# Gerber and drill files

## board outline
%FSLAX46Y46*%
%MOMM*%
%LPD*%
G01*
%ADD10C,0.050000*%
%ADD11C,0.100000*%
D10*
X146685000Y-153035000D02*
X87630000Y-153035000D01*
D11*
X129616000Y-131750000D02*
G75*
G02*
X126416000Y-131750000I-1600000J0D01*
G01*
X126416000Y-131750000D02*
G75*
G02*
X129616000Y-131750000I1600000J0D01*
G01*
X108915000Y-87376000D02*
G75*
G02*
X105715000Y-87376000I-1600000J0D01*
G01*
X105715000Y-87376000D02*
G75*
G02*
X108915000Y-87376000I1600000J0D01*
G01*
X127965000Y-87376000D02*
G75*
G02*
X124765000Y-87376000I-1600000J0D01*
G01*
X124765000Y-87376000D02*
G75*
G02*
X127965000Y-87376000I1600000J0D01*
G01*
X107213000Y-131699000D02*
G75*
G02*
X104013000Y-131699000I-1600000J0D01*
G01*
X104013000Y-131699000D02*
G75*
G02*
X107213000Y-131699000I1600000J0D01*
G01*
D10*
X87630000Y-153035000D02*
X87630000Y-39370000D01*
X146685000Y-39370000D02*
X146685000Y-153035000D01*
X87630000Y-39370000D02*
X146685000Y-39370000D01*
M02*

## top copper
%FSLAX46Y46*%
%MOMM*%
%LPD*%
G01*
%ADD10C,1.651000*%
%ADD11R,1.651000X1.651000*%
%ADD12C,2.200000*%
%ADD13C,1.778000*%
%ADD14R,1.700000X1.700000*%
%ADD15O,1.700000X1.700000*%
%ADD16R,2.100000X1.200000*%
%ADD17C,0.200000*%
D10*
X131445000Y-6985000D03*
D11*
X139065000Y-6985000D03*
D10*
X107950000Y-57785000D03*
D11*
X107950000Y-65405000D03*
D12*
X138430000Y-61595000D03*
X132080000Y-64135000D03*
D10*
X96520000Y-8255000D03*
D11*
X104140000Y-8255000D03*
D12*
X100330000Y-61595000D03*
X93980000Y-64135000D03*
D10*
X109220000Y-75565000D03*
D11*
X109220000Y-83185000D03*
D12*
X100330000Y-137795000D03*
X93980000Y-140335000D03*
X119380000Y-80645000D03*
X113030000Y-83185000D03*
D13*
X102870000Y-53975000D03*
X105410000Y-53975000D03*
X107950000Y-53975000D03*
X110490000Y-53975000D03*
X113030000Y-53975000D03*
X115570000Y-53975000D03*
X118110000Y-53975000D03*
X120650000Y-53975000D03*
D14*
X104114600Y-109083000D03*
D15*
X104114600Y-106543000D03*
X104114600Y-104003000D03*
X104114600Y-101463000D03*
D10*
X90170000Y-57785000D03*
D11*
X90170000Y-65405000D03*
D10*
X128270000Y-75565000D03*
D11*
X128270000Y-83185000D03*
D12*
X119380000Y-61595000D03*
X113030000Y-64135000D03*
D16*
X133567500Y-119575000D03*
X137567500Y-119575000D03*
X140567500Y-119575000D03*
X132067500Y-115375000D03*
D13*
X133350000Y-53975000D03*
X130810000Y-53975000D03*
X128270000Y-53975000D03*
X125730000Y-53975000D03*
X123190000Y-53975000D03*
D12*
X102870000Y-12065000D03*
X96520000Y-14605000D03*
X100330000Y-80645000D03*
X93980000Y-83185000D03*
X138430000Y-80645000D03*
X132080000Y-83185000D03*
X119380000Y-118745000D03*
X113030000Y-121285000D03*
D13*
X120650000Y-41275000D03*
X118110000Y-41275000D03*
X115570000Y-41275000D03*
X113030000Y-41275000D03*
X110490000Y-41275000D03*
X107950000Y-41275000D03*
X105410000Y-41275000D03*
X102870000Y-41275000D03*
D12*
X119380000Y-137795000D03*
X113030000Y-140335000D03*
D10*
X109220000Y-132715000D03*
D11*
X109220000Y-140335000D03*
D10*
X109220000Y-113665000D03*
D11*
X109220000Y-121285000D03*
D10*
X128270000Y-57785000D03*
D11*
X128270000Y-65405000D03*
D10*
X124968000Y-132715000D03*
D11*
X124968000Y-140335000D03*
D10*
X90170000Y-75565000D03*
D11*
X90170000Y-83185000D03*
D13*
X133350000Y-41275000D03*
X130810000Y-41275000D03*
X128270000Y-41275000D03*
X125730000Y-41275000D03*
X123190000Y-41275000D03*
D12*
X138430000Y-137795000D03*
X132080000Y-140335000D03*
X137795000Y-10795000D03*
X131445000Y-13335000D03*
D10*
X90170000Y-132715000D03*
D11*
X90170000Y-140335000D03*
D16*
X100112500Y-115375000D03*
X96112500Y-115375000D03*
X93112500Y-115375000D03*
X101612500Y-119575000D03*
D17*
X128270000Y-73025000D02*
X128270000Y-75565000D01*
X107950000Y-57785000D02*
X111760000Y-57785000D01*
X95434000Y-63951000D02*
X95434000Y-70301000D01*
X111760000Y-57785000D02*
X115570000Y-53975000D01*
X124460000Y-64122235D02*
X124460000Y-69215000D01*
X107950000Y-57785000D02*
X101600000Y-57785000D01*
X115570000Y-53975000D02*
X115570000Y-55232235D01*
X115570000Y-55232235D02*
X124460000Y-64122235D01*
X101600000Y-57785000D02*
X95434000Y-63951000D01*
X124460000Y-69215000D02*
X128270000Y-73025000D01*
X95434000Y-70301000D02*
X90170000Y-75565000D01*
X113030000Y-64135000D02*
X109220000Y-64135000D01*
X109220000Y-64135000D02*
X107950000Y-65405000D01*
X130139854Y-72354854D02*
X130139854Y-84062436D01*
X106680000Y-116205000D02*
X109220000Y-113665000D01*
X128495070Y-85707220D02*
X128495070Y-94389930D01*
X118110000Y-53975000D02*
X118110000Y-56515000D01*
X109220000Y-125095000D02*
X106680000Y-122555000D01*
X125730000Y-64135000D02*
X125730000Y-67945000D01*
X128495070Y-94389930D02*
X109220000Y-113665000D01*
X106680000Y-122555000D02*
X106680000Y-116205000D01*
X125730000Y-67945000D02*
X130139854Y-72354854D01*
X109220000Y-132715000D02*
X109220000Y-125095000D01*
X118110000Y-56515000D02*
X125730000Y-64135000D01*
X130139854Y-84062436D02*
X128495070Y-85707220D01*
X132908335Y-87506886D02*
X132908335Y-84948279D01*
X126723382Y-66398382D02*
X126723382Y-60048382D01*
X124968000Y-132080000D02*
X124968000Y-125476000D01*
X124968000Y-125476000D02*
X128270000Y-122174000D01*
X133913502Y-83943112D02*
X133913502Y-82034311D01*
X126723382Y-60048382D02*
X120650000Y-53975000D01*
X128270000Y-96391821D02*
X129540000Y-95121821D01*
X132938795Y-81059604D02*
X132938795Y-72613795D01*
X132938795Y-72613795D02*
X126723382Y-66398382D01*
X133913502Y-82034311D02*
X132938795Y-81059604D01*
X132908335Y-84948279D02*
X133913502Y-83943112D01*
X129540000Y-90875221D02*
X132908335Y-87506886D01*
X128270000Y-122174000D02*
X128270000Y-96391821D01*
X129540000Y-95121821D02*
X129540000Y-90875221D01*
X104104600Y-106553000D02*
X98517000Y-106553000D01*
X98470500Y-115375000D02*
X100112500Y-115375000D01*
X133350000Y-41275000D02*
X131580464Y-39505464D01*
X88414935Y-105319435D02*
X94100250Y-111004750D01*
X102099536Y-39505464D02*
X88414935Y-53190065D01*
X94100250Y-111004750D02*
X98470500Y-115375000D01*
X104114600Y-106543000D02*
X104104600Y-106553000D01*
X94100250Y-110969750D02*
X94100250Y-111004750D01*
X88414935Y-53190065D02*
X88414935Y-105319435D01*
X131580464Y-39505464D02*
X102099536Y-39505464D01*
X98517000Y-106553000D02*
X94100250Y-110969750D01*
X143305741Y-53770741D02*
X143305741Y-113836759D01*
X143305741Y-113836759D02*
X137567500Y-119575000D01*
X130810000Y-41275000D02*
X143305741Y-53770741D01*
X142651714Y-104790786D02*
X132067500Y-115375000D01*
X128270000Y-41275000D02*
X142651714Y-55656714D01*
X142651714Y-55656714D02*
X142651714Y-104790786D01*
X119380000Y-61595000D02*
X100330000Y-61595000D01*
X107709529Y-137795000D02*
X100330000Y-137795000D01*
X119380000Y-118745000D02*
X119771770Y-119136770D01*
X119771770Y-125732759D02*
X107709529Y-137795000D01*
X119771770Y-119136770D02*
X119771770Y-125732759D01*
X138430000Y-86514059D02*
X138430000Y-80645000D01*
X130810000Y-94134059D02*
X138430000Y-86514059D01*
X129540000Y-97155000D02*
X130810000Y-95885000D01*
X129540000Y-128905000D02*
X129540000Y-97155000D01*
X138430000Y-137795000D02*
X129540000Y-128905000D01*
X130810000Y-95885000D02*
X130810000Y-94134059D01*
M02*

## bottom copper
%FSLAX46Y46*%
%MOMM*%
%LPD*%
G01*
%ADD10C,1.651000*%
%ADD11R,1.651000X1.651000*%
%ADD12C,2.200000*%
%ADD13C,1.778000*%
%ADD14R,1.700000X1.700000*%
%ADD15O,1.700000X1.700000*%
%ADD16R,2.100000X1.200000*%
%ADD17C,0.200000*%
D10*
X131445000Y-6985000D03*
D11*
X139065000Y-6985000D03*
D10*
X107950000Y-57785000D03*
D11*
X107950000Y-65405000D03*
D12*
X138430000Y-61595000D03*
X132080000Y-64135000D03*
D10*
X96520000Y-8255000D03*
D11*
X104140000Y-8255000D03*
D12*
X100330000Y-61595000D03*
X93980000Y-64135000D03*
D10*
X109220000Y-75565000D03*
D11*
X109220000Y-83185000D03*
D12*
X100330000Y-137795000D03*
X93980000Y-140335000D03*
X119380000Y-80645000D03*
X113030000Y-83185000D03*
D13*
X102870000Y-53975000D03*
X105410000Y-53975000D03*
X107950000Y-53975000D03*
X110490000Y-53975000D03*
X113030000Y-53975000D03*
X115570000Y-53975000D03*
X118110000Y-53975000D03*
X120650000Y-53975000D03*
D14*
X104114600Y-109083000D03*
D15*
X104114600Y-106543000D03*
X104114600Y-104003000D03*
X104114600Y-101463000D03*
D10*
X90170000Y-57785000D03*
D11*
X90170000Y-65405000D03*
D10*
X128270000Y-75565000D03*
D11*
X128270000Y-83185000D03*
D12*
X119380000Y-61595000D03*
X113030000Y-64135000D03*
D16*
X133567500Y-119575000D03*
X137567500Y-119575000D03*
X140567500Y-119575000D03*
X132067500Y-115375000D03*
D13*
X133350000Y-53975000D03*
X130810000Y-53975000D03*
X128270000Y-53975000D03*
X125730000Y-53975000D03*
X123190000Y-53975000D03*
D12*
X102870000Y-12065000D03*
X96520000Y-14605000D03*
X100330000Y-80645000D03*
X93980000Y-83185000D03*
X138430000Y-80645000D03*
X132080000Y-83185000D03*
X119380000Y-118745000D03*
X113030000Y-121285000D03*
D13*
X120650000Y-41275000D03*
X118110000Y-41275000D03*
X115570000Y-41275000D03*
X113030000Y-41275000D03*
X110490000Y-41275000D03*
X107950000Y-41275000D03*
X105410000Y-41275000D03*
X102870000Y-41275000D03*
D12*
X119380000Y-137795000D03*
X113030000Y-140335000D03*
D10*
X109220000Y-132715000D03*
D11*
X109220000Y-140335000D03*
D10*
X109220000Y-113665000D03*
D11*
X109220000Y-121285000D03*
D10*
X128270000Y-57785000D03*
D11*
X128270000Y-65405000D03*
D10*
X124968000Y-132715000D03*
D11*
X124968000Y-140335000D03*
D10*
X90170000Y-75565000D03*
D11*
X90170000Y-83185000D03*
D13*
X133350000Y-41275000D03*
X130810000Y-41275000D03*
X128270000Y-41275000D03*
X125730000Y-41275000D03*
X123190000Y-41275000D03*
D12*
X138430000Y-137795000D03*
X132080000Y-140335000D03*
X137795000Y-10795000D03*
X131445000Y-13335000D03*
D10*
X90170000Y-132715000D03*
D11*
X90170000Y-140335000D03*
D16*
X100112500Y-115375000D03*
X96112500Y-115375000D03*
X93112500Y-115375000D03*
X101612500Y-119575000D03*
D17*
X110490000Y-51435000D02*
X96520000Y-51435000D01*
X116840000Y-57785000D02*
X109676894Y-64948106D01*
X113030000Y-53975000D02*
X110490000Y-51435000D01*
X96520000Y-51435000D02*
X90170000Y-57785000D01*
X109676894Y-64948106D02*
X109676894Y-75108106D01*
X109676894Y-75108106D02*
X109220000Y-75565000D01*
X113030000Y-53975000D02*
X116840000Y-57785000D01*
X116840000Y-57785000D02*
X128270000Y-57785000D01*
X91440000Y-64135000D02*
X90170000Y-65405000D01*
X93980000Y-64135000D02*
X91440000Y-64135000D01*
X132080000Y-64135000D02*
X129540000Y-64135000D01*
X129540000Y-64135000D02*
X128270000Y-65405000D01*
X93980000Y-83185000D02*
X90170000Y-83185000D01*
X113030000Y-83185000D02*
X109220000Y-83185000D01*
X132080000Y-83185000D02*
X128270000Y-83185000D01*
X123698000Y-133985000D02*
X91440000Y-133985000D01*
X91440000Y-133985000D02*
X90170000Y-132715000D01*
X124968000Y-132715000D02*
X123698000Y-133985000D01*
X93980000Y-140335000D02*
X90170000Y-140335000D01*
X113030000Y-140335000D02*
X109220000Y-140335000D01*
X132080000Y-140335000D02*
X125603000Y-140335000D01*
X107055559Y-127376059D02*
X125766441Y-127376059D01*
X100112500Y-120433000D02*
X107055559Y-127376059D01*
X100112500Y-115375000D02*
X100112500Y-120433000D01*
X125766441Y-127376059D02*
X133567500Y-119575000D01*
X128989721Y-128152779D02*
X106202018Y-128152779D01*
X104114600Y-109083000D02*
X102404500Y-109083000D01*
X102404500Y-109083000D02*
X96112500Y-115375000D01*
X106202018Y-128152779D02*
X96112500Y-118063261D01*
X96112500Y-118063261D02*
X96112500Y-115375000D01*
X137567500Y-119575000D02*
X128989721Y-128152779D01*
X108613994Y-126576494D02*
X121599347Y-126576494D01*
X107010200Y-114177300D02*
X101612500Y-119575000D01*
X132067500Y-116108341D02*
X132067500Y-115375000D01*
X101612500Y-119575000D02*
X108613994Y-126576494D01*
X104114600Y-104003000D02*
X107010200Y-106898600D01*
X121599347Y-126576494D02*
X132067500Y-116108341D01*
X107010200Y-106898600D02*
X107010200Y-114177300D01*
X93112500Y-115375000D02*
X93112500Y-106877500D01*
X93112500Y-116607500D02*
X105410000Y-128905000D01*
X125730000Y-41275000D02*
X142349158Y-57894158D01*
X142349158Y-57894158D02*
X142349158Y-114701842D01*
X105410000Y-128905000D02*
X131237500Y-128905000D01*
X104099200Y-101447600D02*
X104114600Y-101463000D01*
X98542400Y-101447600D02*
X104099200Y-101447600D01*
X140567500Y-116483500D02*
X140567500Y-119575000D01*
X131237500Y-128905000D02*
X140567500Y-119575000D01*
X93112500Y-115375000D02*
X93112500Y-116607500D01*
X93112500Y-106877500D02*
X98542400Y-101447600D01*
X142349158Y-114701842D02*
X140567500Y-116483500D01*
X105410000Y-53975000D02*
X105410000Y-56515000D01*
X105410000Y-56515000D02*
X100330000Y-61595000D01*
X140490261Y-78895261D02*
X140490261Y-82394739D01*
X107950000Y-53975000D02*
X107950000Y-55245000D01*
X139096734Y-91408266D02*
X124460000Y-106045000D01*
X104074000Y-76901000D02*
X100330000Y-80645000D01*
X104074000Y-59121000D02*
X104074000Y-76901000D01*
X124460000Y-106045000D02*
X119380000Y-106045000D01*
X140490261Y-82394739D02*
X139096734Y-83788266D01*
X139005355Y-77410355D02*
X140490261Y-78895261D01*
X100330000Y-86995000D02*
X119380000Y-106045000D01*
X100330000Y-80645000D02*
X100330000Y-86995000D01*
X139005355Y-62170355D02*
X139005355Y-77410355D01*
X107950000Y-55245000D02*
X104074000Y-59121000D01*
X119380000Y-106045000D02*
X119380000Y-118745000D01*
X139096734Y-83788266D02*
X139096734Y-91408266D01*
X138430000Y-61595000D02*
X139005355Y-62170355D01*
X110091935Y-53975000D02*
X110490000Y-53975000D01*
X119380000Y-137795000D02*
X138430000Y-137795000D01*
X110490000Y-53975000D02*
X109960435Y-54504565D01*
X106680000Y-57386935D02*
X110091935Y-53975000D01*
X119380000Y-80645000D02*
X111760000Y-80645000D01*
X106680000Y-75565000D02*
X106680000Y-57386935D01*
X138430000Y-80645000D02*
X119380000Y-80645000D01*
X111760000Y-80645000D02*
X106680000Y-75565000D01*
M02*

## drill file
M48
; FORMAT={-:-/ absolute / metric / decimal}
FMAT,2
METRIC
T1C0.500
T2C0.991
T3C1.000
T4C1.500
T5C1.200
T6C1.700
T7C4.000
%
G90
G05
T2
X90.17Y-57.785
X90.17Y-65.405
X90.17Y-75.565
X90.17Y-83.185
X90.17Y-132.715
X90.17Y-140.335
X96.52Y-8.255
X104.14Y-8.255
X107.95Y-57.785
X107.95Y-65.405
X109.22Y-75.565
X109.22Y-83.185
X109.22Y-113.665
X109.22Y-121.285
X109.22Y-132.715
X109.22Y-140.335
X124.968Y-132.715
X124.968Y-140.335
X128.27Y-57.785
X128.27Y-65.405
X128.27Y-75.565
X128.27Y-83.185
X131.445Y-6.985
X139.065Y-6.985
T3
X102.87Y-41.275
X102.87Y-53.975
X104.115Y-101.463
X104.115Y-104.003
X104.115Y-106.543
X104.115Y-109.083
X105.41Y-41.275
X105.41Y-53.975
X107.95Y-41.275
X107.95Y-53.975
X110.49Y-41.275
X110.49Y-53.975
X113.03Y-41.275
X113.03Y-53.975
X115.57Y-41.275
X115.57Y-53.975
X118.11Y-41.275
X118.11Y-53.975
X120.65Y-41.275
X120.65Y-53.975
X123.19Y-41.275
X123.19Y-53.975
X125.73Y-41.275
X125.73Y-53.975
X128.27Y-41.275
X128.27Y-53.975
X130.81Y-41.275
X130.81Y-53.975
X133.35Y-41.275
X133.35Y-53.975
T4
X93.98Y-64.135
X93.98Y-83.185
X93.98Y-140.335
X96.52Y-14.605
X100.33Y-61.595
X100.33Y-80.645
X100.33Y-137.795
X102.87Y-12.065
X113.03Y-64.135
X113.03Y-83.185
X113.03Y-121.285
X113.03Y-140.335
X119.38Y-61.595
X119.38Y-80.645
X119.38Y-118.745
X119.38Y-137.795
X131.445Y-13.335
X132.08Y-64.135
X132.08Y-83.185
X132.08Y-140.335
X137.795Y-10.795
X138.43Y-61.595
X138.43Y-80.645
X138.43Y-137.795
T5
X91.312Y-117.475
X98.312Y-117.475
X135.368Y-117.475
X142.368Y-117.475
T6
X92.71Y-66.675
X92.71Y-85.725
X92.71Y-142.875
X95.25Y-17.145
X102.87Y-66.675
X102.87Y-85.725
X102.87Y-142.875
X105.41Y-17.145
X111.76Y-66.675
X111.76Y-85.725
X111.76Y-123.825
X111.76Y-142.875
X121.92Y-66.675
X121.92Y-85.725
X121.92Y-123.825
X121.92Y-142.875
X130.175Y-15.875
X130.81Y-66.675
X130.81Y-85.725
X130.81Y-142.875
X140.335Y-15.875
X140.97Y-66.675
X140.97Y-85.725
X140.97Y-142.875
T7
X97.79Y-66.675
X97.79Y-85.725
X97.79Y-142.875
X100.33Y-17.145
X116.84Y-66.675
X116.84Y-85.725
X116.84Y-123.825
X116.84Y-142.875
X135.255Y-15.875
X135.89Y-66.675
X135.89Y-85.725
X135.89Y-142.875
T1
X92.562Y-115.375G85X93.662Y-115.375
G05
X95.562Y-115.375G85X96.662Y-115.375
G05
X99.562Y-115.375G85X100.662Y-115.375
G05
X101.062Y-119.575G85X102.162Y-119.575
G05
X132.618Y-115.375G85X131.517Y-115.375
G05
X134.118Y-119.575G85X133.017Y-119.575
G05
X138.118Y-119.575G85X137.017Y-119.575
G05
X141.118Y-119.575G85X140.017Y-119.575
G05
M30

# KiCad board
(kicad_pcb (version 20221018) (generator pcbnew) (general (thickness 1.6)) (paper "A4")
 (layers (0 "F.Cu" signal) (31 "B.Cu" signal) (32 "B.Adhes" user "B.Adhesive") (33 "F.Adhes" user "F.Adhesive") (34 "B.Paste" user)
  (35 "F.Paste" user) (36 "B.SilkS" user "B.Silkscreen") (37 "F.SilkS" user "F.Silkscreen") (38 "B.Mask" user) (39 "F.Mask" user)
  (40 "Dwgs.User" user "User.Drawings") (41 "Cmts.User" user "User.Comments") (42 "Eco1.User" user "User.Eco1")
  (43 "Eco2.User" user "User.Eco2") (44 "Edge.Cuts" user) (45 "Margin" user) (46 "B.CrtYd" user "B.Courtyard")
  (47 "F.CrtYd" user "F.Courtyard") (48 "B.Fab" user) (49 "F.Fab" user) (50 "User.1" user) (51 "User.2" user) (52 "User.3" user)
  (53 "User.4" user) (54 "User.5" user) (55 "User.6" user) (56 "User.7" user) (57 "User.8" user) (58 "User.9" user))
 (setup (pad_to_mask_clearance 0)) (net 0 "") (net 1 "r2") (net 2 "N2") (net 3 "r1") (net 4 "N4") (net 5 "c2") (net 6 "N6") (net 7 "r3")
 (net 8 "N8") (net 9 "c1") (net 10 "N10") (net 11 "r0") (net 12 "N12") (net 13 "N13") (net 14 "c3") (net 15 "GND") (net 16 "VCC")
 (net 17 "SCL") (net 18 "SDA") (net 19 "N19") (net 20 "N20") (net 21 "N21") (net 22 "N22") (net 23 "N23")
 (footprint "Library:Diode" (layer "F.Cu") (at 135.255 6.985)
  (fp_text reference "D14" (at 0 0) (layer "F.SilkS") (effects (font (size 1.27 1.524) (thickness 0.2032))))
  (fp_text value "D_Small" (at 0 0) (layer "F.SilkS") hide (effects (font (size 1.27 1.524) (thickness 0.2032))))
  (pad "1" thru_hole circle (at -3.81 0) (size 1.651 1.651) (drill 0.9906) (layers "*.Cu" "*.SilkS" "*.Mask") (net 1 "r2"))
  (pad "2" thru_hole rect (at 3.81 0) (size 1.651 1.651) (drill 0.9906) (layers "*.Cu" "*.SilkS" "*.Mask") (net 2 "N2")))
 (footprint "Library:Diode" (layer "F.Cu") (at 107.95 61.595 -90)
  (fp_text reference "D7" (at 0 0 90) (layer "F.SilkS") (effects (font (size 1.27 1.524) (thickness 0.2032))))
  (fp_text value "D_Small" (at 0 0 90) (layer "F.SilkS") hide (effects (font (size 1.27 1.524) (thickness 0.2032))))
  (pad "1" thru_hole circle (at -3.81 0 270) (size 1.651 1.651) (drill 0.9906) (layers "*.Cu" "*.SilkS" "*.Mask") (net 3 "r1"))
  (pad "2" thru_hole rect (at 3.81 0 270) (size 1.651 1.651) (drill 0.9906) (layers "*.Cu" "*.SilkS" "*.Mask") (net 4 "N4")))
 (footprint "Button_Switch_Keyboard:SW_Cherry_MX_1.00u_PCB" (layer "F.Cu") (at 138.43 61.595)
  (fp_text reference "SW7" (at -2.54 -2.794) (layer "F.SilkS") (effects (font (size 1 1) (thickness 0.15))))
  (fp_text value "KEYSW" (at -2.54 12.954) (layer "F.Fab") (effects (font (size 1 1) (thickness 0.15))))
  (pad "" np_thru_hole circle (at -7.62 5.08) (size 1.7 1.7) (drill 1.7) (layers "*.Cu" "*.Mask"))
  (pad "" np_thru_hole circle (at -2.54 5.08) (size 4 4) (drill 4) (layers "*.Cu" "*.Mask"))
  (pad "" np_thru_hole circle (at 2.54 5.08) (size 1.7 1.7) (drill 1.7) (layers "*.Cu" "*.Mask"))
  (pad "1" thru_hole circle (at 0 0) (size 2.2 2.2) (drill 1.5) (layers "*.Cu" "*.Mask") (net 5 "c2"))
  (pad "2" thru_hole circle (at -6.35 2.54) (size 2.2 2.2) (drill 1.5) (layers "*.Cu" "*.Mask") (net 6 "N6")))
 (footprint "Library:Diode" (layer "F.Cu") (at 100.33 8.255)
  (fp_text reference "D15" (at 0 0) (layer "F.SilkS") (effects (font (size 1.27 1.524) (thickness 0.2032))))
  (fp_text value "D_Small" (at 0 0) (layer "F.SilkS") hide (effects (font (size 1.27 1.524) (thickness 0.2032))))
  (pad "1" thru_hole circle (at -3.81 0) (size 1.651 1.651) (drill 0.9906) (layers "*.Cu" "*.SilkS" "*.Mask") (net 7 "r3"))
  (pad "2" thru_hole rect (at 3.81 0) (size 1.651 1.651) (drill 0.9906) (layers "*.Cu" "*.SilkS" "*.Mask") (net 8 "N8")))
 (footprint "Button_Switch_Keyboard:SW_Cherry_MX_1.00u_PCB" (layer "F.Cu") (at 100.33 61.595)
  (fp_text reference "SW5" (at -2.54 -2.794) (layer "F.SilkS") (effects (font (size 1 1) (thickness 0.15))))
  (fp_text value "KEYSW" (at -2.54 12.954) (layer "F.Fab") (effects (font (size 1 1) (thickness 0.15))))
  (pad "" np_thru_hole circle (at -7.62 5.08) (size 1.7 1.7) (drill 1.7) (layers "*.Cu" "*.Mask"))
  (pad "" np_thru_hole circle (at -2.54 5.08) (size 4 4) (drill 4) (layers "*.Cu" "*.Mask"))
  (pad "" np_thru_hole circle (at 2.54 5.08) (size 1.7 1.7) (drill 1.7) (layers "*.Cu" "*.Mask"))
  (pad "1" thru_hole circle (at 0 0) (size 2.2 2.2) (drill 1.5) (layers "*.Cu" "*.Mask") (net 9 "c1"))
  (pad "2" thru_hole circle (at -6.35 2.54) (size 2.2 2.2) (drill 1.5) (layers "*.Cu" "*.Mask") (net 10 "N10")))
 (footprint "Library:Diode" (layer "F.Cu") (at 109.22 79.375 -90)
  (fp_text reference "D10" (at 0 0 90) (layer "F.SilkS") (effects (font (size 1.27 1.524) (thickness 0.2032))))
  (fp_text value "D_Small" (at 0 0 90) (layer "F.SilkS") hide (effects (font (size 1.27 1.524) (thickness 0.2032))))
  (pad "1" thru_hole circle (at -3.81 0 270) (size 1.651 1.651) (drill 0.9906) (layers "*.Cu" "*.SilkS" "*.Mask") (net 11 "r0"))
  (pad "2" thru_hole rect (at 3.81 0 270) (size 1.651 1.651) (drill 0.9906) (layers "*.Cu" "*.SilkS" "*.Mask") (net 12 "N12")))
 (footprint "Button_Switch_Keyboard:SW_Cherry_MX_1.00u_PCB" (layer "F.Cu") (at 100.33 137.795)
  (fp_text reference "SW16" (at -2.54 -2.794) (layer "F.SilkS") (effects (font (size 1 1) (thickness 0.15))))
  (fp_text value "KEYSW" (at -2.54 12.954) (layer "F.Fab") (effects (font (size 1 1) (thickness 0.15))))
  (pad "" np_thru_hole circle (at -7.62 5.08) (size 1.7 1.7) (drill 1.7) (layers "*.Cu" "*.Mask"))
  (pad "" np_thru_hole circle (at -2.54 5.08) (size 4 4) (drill 4) (layers "*.Cu" "*.Mask"))
  (pad "" np_thru_hole circle (at 2.54 5.08) (size 1.7 1.7) (drill 1.7) (layers "*.Cu" "*.Mask"))
  (pad "1" thru_hole circle (at 0 0) (size 2.2 2.2) (drill 1.5) (layers "*.Cu" "*.Mask") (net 5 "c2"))
  (pad "2" thru_hole circle (at -6.35 2.54) (size 2.2 2.2) (drill 1.5) (layers "*.Cu" "*.Mask") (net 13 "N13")))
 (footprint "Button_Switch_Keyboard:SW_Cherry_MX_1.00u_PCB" (layer "F.Cu") (at 119.38 80.645)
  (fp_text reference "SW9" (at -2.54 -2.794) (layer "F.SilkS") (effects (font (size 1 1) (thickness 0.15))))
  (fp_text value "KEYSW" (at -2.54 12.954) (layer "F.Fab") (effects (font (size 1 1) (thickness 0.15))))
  (pad "" np_thru_hole circle (at -7.62 5.08) (size 1.7 1.7) (drill 1.7) (layers "*.Cu" "*.Mask"))
  (pad "" np_thru_hole circle (at -2.54 5.08) (size 4 4) (drill 4) (layers "*.Cu" "*.Mask"))
  (pad "" np_thru_hole circle (at 2.54 5.08) (size 1.7 1.7) (drill 1.7) (layers "*.Cu" "*.Mask"))
  (pad "1" thru_hole circle (at 0 0) (size 2.2 2.2) (drill 1.5) (layers "*.Cu" "*.Mask") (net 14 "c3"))
  (pad "2" thru_hole circle (at -6.35 2.54) (size 2.2 2.2) (drill 1.5) (layers "*.Cu" "*.Mask") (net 12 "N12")))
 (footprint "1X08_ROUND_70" (layer "F.Cu") (at 111.76 53.975)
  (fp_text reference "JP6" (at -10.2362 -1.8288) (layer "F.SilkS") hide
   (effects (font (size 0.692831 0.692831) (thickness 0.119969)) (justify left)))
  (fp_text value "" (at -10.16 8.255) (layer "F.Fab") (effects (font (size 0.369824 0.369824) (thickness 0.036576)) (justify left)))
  (pad "1" thru_hole circle (at -8.89 0 90) (size 1.778 1.778) (drill 1) (layers "*.Cu" "*.Mask") (solder_mask_margin 0.0508))
  (pad "2" thru_hole circle (at -6.35 0 90) (size 1.778 1.778) (drill 1) (layers "*.Cu" "*.Mask") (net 9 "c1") (solder_mask_margin 0.0508))
  (pad "3" thru_hole circle (at -3.81 0 90) (size 1.778 1.778) (drill 1) (layers "*.Cu" "*.Mask") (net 5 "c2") (solder_mask_margin 0.0508))
  (pad "4" thru_hole circle (at -1.27 0 90) (size 1.778 1.778) (drill 1) (layers "*.Cu" "*.Mask") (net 14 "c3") (solder_mask_margin 0.0508))
  (pad "5" thru_hole circle (at 1.27 0 90) (size 1.778 1.778) (drill 1) (layers "*.Cu" "*.Mask") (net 11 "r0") (solder_mask_margin 0.0508))
  (pad "6" thru_hole circle (at 3.81 0 90) (size 1.778 1.778) (drill 1) (layers "*.Cu" "*.Mask") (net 3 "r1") (solder_mask_margin 0.0508))
  (pad "7" thru_hole circle (at 6.35 0 90) (size 1.778 1.778) (drill 1) (layers "*.Cu" "*.Mask") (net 1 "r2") (solder_mask_margin 0.0508))
  (pad "8" thru_hole circle (at 8.89 0 90) (size 1.778 1.778) (drill 1) (layers "*.Cu" "*.Mask") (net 7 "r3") (solder_mask_margin 0.0508)))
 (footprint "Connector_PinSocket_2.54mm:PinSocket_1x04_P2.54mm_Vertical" (layer "F.Cu") (at 104.1146 109.083 180)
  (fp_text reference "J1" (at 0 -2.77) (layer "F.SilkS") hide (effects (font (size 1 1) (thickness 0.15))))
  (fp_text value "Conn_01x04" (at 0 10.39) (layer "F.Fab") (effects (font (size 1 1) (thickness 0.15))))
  (pad "1" thru_hole rect (at 0 0 180) (size 1.7 1.7) (drill 1) (layers "*.Cu" "*.Mask") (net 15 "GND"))
  (pad "2" thru_hole oval (at 0 2.54 180) (size 1.7 1.7) (drill 1) (layers "*.Cu" "*.Mask") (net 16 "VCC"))
  (pad "3" thru_hole oval (at 0 5.08 180) (size 1.7 1.7) (drill 1) (layers "*.Cu" "*.Mask") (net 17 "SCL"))
  (pad "4" thru_hole oval (at 0 7.62 180) (size 1.7 1.7) (drill 1) (layers "*.Cu" "*.Mask") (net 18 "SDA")))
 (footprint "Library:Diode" (layer "F.Cu") (at 90.17 61.595 -90)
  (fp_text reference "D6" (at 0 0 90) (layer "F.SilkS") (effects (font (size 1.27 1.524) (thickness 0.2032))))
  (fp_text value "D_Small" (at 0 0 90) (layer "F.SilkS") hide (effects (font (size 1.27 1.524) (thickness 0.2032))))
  (pad "1" thru_hole circle (at -3.81 0 270) (size 1.651 1.651) (drill 0.9906) (layers "*.Cu" "*.SilkS" "*.Mask") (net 11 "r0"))
  (pad "2" thru_hole rect (at 3.81 0 270) (size 1.651 1.651) (drill 0.9906) (layers "*.Cu" "*.SilkS" "*.Mask") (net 10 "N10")))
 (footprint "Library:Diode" (layer "F.Cu") (at 128.27 79.375 -90)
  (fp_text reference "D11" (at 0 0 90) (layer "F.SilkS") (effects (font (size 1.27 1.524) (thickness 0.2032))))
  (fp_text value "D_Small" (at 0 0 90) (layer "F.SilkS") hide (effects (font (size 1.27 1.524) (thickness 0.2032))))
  (pad "1" thru_hole circle (at -3.81 0 270) (size 1.651 1.651) (drill 0.9906) (layers "*.Cu" "*.SilkS" "*.Mask") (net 3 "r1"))
  (pad "2" thru_hole rect (at 3.81 0 270) (size 1.651 1.651) (drill 0.9906) (layers "*.Cu" "*.SilkS" "*.Mask") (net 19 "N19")))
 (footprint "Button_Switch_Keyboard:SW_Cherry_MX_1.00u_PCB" (layer "F.Cu") (at 119.38 61.595)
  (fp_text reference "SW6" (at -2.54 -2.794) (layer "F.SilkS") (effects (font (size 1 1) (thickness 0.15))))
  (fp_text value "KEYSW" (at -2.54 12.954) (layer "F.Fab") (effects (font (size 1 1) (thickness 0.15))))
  (pad "" np_thru_hole circle (at -7.62 5.08) (size 1.7 1.7) (drill 1.7) (layers "*.Cu" "*.Mask"))
  (pad "" np_thru_hole circle (at -2.54 5.08) (size 4 4) (drill 4) (layers "*.Cu" "*.Mask"))
  (pad "" np_thru_hole circle (at 2.54 5.08) (size 1.7 1.7) (drill 1.7) (layers "*.Cu" "*.Mask"))
  (pad "1" thru_hole circle (at 0 0) (size 2.2 2.2) (drill 1.5) (layers "*.Cu" "*.Mask") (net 9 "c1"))
  (pad "2" thru_hole circle (at -6.35 2.54) (size 2.2 2.2) (drill 1.5) (layers "*.Cu" "*.Mask") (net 4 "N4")))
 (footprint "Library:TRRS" (layer "F.Cu") (at 143.8675 117.475 -90)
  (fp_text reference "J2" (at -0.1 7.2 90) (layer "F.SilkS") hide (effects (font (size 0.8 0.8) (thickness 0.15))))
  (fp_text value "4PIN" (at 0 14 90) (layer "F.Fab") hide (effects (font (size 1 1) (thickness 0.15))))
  (pad "" np_thru_hole circle (at 0 1.5 270) (size 1.2 1.2) (drill 1.2) (layers "*.Cu" "*.Mask" "F.SilkS"))
  (pad "" np_thru_hole circle (at 0 8.5 270) (size 1.2 1.2) (drill 1.2) (layers "*.Cu" "*.Mask" "F.SilkS"))
  (pad "1" thru_hole rect (at 2.1 10.3 270) (size 1.2 2.1) (drill oval 0.5 1.6) (layers "*.Cu" "*.Mask" "F.SilkS") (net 16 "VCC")
   (clearance 0.15))
  (pad "2" thru_hole rect (at 2.1 6.3 270) (size 1.2 2.1) (drill oval 0.5 1.6) (layers "*.Cu" "*.Mask" "F.SilkS") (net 15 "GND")
   (clearance 0.15))
  (pad "3" thru_hole rect (at 2.1 3.3 270) (size 1.2 2.1) (drill oval 0.5 1.6) (layers "*.Cu" "*.Mask" "F.SilkS") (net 18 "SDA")
   (clearance 0.15))
  (pad "4" thru_hole rect (at -2.1 11.8 270) (size 1.2 2.1) (drill oval 0.5 1.6) (layers "*.Cu" "*.Mask" "F.SilkS") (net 17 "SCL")
   (clearance 0.15)))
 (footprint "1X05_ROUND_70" (layer "F.Cu") (at 128.27 53.975 180)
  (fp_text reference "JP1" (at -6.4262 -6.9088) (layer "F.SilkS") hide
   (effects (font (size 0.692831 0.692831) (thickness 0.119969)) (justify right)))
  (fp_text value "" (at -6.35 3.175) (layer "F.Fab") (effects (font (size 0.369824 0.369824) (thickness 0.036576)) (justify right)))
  (pad "1" thru_hole circle (at -5.08 0 270) (size 1.778 1.778) (drill 1) (layers "*.Cu" "*.Mask") (solder_mask_margin 0.0508))
  (pad "2" thru_hole circle (at -2.54 0 270) (size 1.778 1.778) (drill 1) (layers "*.Cu" "*.Mask") (solder_mask_margin 0.0508))
  (pad "3" thru_hole circle (at 0 0 270) (size 1.778 1.778) (drill 1) (layers "*.Cu" "*.Mask") (solder_mask_margin 0.0508))
  (pad "4" thru_hole circle (at 2.54 0 270) (size 1.778 1.778) (drill 1) (layers "*.Cu" "*.Mask") (solder_mask_margin 0.0508))
  (pad "5" thru_hole circle (at 5.08 0 270) (size 1.778 1.778) (drill 1) (layers "*.Cu" "*.Mask") (solder_mask_margin 0.0508)))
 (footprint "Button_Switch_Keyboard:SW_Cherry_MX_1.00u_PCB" (layer "F.Cu") (at 102.87 12.065)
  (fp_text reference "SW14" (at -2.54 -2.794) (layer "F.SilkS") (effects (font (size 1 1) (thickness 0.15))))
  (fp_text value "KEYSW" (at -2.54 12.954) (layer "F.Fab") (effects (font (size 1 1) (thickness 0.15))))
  (pad "" np_thru_hole circle (at -7.62 5.08) (size 1.7 1.7) (drill 1.7) (layers "*.Cu" "*.Mask"))
  (pad "" np_thru_hole circle (at -2.54 5.08) (size 4 4) (drill 4) (layers "*.Cu" "*.Mask"))
  (pad "" np_thru_hole circle (at 2.54 5.08) (size 1.7 1.7) (drill 1.7) (layers "*.Cu" "*.Mask"))
  (pad "1" thru_hole circle (at 0 0) (size 2.2 2.2) (drill 1.5) (layers "*.Cu" "*.Mask") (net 9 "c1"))
  (pad "2" thru_hole circle (at -6.35 2.54) (size 2.2 2.2) (drill 1.5) (layers "*.Cu" "*.Mask") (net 8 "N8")))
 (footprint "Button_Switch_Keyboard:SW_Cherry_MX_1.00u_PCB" (layer "F.Cu") (at 100.33 80.645)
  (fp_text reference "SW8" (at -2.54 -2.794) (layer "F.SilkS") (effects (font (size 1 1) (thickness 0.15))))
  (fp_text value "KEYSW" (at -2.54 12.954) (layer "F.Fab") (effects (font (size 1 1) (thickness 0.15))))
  (pad "" np_thru_hole circle (at -7.62 5.08) (size 1.7 1.7) (drill 1.7) (layers "*.Cu" "*.Mask"))
  (pad "" np_thru_hole circle (at -2.54 5.08) (size 4 4) (drill 4) (layers "*.Cu" "*.Mask"))
  (pad "" np_thru_hole circle (at 2.54 5.08) (size 1.7 1.7) (drill 1.7) (layers "*.Cu" "*.Mask"))
  (pad "1" thru_hole circle (at 0 0) (size 2.2 2.2) (drill 1.5) (layers "*.Cu" "*.Mask") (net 5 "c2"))
  (pad "2" thru_hole circle (at -6.35 2.54) (size 2.2 2.2) (drill 1.5) (layers "*.Cu" "*.Mask") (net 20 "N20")))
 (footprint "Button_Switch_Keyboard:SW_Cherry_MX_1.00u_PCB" (layer "F.Cu") (at 138.43 80.645)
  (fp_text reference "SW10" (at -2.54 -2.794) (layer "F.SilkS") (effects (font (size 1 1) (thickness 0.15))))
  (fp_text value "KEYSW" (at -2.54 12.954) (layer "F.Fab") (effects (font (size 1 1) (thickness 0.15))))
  (pad "" np_thru_hole circle (at -7.62 5.08) (size 1.7 1.7) (drill 1.7) (layers "*.Cu" "*.Mask"))
  (pad "" np_thru_hole circle (at -2.54 5.08) (size 4 4) (drill 4) (layers "*.Cu" "*.Mask"))
  (pad "" np_thru_hole circle (at 2.54 5.08) (size 1.7 1.7) (drill 1.7) (layers "*.Cu" "*.Mask"))
  (pad "1" thru_hole circle (at 0 0) (size 2.2 2.2) (drill 1.5) (layers "*.Cu" "*.Mask") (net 14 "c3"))
  (pad "2" thru_hole circle (at -6.35 2.54) (size 2.2 2.2) (drill 1.5) (layers "*.Cu" "*.Mask") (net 19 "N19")))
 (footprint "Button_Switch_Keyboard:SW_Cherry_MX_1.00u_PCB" (layer "F.Cu") (at 119.38 118.745)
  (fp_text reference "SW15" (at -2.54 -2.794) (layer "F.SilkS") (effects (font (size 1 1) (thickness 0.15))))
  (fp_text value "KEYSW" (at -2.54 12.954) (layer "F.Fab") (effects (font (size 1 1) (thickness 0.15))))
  (pad "" np_thru_hole circle (at -7.62 5.08) (size 1.7 1.7) (drill 1.7) (layers "*.Cu" "*.Mask"))
  (pad "" np_thru_hole circle (at -2.54 5.08) (size 4 4) (drill 4) (layers "*.Cu" "*.Mask"))
  (pad "" np_thru_hole circle (at 2.54 5.08) (size 1.7 1.7) (drill 1.7) (layers "*.Cu" "*.Mask"))
  (pad "1" thru_hole circle (at 0 0) (size 2.2 2.2) (drill 1.5) (layers "*.Cu" "*.Mask") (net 5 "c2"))
  (pad "2" thru_hole circle (at -6.35 2.54) (size 2.2 2.2) (drill 1.5) (layers "*.Cu" "*.Mask") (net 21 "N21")))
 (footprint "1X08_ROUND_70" (layer "F.Cu") (at 111.76 41.275 180)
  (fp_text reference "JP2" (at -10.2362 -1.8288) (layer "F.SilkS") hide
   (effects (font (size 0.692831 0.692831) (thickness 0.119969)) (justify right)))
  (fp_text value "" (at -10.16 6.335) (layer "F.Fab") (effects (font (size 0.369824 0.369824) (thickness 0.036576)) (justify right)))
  (pad "1" thru_hole circle (at -8.89 0 270) (size 1.778 1.778) (drill 1) (layers "*.Cu" "*.Mask") (solder_mask_margin 0.0508))
  (pad "2" thru_hole circle (at -6.35 0 270) (size 1.778 1.778) (drill 1) (layers "*.Cu" "*.Mask") (solder_mask_margin 0.0508))
  (pad "3" thru_hole circle (at -3.81 0 270) (size 1.778 1.778) (drill 1) (layers "*.Cu" "*.Mask") (solder_mask_margin 0.0508))
  (pad "4" thru_hole circle (at -1.27 0 270) (size 1.778 1.778) (drill 1) (layers "*.Cu" "*.Mask") (solder_mask_margin 0.0508))
  (pad "5" thru_hole circle (at 1.27 0 270) (size 1.778 1.778) (drill 1) (layers "*.Cu" "*.Mask") (solder_mask_margin 0.0508))
  (pad "6" thru_hole circle (at 3.81 0 270) (size 1.778 1.778) (drill 1) (layers "*.Cu" "*.Mask") (solder_mask_margin 0.0508))
  (pad "7" thru_hole circle (at 6.35 0 270) (size 1.778 1.778) (drill 1) (layers "*.Cu" "*.Mask") (solder_mask_margin 0.0508))
  (pad "8" thru_hole circle (at 8.89 0 270) (size 1.778 1.778) (drill 1) (layers "*.Cu" "*.Mask") (solder_mask_margin 0.0508)))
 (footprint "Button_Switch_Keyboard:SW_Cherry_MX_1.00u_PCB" (layer "F.Cu") (at 119.38 137.795)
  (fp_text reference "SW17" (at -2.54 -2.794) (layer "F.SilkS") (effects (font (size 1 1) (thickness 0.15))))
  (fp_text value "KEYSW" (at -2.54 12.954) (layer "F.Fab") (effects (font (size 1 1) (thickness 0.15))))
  (pad "" np_thru_hole circle (at -7.62 5.08) (size 1.7 1.7) (drill 1.7) (layers "*.Cu" "*.Mask"))
  (pad "" np_thru_hole circle (at -2.54 5.08) (size 4 4) (drill 4) (layers "*.Cu" "*.Mask"))
  (pad "" np_thru_hole circle (at 2.54 5.08) (size 1.7 1.7) (drill 1.7) (layers "*.Cu" "*.Mask"))
  (pad "1" thru_hole circle (at 0 0) (size 2.2 2.2) (drill 1.5) (layers "*.Cu" "*.Mask") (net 14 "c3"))
  (pad "2" thru_hole circle (at -6.35 2.54) (size 2.2 2.2) (drill 1.5) (layers "*.Cu" "*.Mask") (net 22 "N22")))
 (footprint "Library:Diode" (layer "F.Cu") (at 109.22 136.525 -90)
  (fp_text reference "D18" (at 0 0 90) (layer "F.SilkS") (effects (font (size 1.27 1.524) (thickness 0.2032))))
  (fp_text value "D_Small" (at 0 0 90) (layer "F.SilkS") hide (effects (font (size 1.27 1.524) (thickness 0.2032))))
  (pad "1" thru_hole circle (at -3.81 0 270) (size 1.651 1.651) (drill 0.9906) (layers "*.Cu" "*.SilkS" "*.Mask") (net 1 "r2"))
  (pad "2" thru_hole rect (at 3.81 0 270) (size 1.651 1.651) (drill 0.9906) (layers "*.Cu" "*.SilkS" "*.Mask") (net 22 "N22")))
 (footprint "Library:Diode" (layer "F.Cu") (at 109.22 117.475 -90)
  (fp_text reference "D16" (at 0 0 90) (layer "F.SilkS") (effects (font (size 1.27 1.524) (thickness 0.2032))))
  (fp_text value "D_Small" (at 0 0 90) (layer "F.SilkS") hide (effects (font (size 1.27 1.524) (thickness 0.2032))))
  (pad "1" thru_hole circle (at -3.81 0 270) (size 1.651 1.651) (drill 0.9906) (layers "*.Cu" "*.SilkS" "*.Mask") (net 1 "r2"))
  (pad "2" thru_hole rect (at 3.81 0 270) (size 1.651 1.651) (drill 0.9906) (layers "*.Cu" "*.SilkS" "*.Mask") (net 21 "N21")))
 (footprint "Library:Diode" (layer "F.Cu") (at 128.27 61.595 -90)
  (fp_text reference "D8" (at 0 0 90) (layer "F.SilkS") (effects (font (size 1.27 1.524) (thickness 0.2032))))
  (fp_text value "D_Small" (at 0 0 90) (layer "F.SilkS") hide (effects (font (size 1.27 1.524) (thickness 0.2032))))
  (pad "1" thru_hole circle (at -3.81 0 270) (size 1.651 1.651) (drill 0.9906) (layers "*.Cu" "*.SilkS" "*.Mask") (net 11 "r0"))
  (pad "2" thru_hole rect (at 3.81 0 270) (size 1.651 1.651) (drill 0.9906) (layers "*.Cu" "*.SilkS" "*.Mask") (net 6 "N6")))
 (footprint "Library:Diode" (layer "F.Cu") (at 124.968 136.525 -90)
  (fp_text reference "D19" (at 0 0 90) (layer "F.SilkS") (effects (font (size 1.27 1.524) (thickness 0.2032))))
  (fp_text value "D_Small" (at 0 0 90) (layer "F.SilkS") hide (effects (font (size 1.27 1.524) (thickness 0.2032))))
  (pad "1" thru_hole circle (at -3.81 0 270) (size 1.651 1.651) (drill 0.9906) (layers "*.Cu" "*.SilkS" "*.Mask") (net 7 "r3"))
  (pad "2" thru_hole rect (at 3.81 0 270) (size 1.651 1.651) (drill 0.9906) (layers "*.Cu" "*.SilkS" "*.Mask") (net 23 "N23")))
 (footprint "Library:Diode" (layer "F.Cu") (at 90.17 79.375 -90)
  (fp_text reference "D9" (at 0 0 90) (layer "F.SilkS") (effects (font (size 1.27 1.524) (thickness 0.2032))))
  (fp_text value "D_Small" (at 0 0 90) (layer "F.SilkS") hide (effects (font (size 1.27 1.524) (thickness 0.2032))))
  (pad "1" thru_hole circle (at -3.81 0 270) (size 1.651 1.651) (drill 0.9906) (layers "*.Cu" "*.SilkS" "*.Mask") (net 3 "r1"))
  (pad "2" thru_hole rect (at 3.81 0 270) (size 1.651 1.651) (drill 0.9906) (layers "*.Cu" "*.SilkS" "*.Mask") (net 20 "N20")))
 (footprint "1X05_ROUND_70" (layer "F.Cu") (at 128.27 41.275 180)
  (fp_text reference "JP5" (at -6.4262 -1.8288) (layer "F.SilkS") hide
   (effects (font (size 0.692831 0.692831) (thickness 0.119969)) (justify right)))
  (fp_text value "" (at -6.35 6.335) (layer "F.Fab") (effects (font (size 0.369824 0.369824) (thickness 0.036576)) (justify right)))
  (pad "1" thru_hole circle (at -5.08 0 270) (size 1.778 1.778) (drill 1) (layers "*.Cu" "*.Mask") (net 16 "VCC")
   (solder_mask_margin 0.0508))
  (pad "2" thru_hole circle (at -2.54 0 270) (size 1.778 1.778) (drill 1) (layers "*.Cu" "*.Mask") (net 15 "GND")
   (solder_mask_margin 0.0508))
  (pad "3" thru_hole circle (at 0 0 270) (size 1.778 1.778) (drill 1) (layers "*.Cu" "*.Mask") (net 17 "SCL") (solder_mask_margin 0.0508))
  (pad "4" thru_hole circle (at 2.54 0 270) (size 1.778 1.778) (drill 1) (layers "*.Cu" "*.Mask") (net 18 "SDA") (solder_mask_margin 0.0508))
  (pad "5" thru_hole circle (at 5.08 0 270) (size 1.778 1.778) (drill 1) (layers "*.Cu" "*.Mask") (solder_mask_margin 0.0508)))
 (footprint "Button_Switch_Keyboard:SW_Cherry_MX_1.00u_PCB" (layer "F.Cu") (at 138.43 137.795)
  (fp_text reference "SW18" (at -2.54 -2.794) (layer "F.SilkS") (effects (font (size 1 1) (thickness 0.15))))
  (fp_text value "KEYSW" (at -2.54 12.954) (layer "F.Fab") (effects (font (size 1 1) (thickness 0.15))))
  (pad "" np_thru_hole circle (at -7.62 5.08) (size 1.7 1.7) (drill 1.7) (layers "*.Cu" "*.Mask"))
  (pad "" np_thru_hole circle (at -2.54 5.08) (size 4 4) (drill 4) (layers "*.Cu" "*.Mask"))
  (pad "" np_thru_hole circle (at 2.54 5.08) (size 1.7 1.7) (drill 1.7) (layers "*.Cu" "*.Mask"))
  (pad "1" thru_hole circle (at 0 0) (size 2.2 2.2) (drill 1.5) (layers "*.Cu" "*.Mask") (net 14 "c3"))
  (pad "2" thru_hole circle (at -6.35 2.54) (size 2.2 2.2) (drill 1.5) (layers "*.Cu" "*.Mask") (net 23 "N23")))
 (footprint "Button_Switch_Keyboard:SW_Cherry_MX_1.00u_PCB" (layer "F.Cu") (at 137.795 10.795)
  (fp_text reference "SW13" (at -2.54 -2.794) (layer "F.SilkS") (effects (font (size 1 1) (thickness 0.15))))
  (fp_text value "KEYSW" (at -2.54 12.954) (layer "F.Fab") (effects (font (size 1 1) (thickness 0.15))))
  (pad "" np_thru_hole circle (at -7.62 5.08) (size 1.7 1.7) (drill 1.7) (layers "*.Cu" "*.Mask"))
  (pad "" np_thru_hole circle (at -2.54 5.08) (size 4 4) (drill 4) (layers "*.Cu" "*.Mask"))
  (pad "" np_thru_hole circle (at 2.54 5.08) (size 1.7 1.7) (drill 1.7) (layers "*.Cu" "*.Mask"))
  (pad "1" thru_hole circle (at 0 0) (size 2.2 2.2) (drill 1.5) (layers "*.Cu" "*.Mask") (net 9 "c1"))
  (pad "2" thru_hole circle (at -6.35 2.54) (size 2.2 2.2) (drill 1.5) (layers "*.Cu" "*.Mask") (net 2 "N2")))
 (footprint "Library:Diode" (layer "F.Cu") (at 90.17 136.525 -90)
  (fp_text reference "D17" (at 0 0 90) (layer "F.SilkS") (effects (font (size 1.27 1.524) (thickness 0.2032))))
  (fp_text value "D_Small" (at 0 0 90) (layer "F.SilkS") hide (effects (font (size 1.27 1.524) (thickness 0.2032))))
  (pad "1" thru_hole circle (at -3.81 0 270) (size 1.651 1.651) (drill 0.9906) (layers "*.Cu" "*.SilkS" "*.Mask") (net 7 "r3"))
  (pad "2" thru_hole rect (at 3.81 0 270) (size 1.651 1.651) (drill 0.9906) (layers "*.Cu" "*.SilkS" "*.Mask") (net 13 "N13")))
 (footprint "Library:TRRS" (layer "F.Cu") (at 89.8125 117.475 90)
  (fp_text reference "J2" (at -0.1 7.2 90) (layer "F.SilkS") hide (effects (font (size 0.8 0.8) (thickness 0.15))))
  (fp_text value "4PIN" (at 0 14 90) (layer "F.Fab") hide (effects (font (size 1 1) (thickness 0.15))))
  (pad "" np_thru_hole circle (at 0 1.5 90) (size 1.2 1.2) (drill 1.2) (layers "*.Cu" "*.Mask" "F.SilkS"))
  (pad "" np_thru_hole circle (at 0 8.5 90) (size 1.2 1.2) (drill 1.2) (layers "*.Cu" "*.Mask" "F.SilkS"))
  (pad "1" thru_hole rect (at 2.1 10.3 90) (size 1.2 2.1) (drill oval 0.5 1.6) (layers "*.Cu" "*.Mask" "F.SilkS") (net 16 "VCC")
   (clearance 0.15))
  (pad "2" thru_hole rect (at 2.1 6.3 90) (size 1.2 2.1) (drill oval 0.5 1.6) (layers "*.Cu" "*.Mask" "F.SilkS") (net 15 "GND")
   (clearance 0.15))
  (pad "3" thru_hole rect (at 2.1 3.3 90) (size 1.2 2.1) (drill oval 0.5 1.6) (layers "*.Cu" "*.Mask" "F.SilkS") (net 18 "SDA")
   (clearance 0.15))
  (pad "4" thru_hole rect (at -2.1 11.8 90) (size 1.2 2.1) (drill oval 0.5 1.6) (layers "*.Cu" "*.Mask" "F.SilkS") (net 17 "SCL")
   (clearance 0.15)))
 (gr_line (start 146.685 153.035) (end 87.63 153.035) (stroke (width 0.05) (type default)) (layer "Edge.Cuts"))
 (gr_circle (center 128.016 131.75) (end 129.616 131.75) (stroke (width 0.1) (type default)) (fill none) (layer "Edge.Cuts"))
 (gr_circle (center 107.315 87.376) (end 108.915 87.376) (stroke (width 0.1) (type default)) (fill none) (layer "Edge.Cuts"))
 (gr_circle (center 126.365 87.376) (end 127.965 87.376) (stroke (width 0.1) (type default)) (fill none) (layer "Edge.Cuts"))
 (gr_circle (center 105.613 131.699) (end 107.213 131.699) (stroke (width 0.1) (type default)) (fill none) (layer "Edge.Cuts"))
 (gr_line (start 87.63 153.035) (end 87.63 39.37) (stroke (width 0.05) (type default)) (layer "Edge.Cuts"))
 (gr_line (start 146.685 39.37) (end 146.685 153.035) (stroke (width 0.05) (type default)) (layer "Edge.Cuts"))
 (gr_line (start 87.63 39.37) (end 146.685 39.37) (stroke (width 0.05) (type default)) (layer "Edge.Cuts"))
 (segment (start 110.49 51.435) (end 96.52 51.435) (width 0.2) (layer "B.Cu") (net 11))
 (segment (start 116.84 57.785) (end 109.676894 64.948106) (width 0.2) (layer "B.Cu") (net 11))
 (segment (start 113.03 53.975) (end 110.49 51.435) (width 0.2) (layer "B.Cu") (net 11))
 (segment (start 96.52 51.435) (end 90.17 57.785) (width 0.2) (layer "B.Cu") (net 11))
 (segment (start 109.676894 64.948106) (end 109.676894 75.108106) (width 0.2) (layer "B.Cu") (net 11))
 (segment (start 109.676894 75.108106) (end 109.22 75.565) (width 0.2) (layer "B.Cu") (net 11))
 (segment (start 113.03 53.975) (end 116.84 57.785) (width 0.2) (layer "B.Cu") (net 11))
 (segment (start 116.84 57.785) (end 128.27 57.785) (width 0.2) (layer "B.Cu") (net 11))
 (segment (start 91.44 64.135) (end 90.17 65.405) (width 0.2) (layer "B.Cu") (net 10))
 (segment (start 93.98 64.135) (end 91.44 64.135) (width 0.2) (layer "B.Cu") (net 10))
 (segment (start 128.27 73.025) (end 128.27 75.565) (width 0.2) (layer "F.Cu") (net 3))
 (segment (start 107.95 57.785) (end 111.76 57.785) (width 0.2) (layer "F.Cu") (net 3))
 (segment (start 95.434 63.951) (end 95.434 70.301) (width 0.2) (layer "F.Cu") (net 3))
 (segment (start 111.76 57.785) (end 115.57 53.975) (width 0.2) (layer "F.Cu") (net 3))
 (segment (start 124.46 64.122235) (end 124.46 69.215) (width 0.2) (layer "F.Cu") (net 3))
 (segment (start 107.95 57.785) (end 101.6 57.785) (width 0.2) (layer "F.Cu") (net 3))
 (segment (start 115.57 53.975) (end 115.57 55.232235) (width 0.2) (layer "F.Cu") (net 3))
 (segment (start 115.57 55.232235) (end 124.46 64.122235) (width 0.2) (layer "F.Cu") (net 3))
 (segment (start 101.6 57.785) (end 95.434 63.951) (width 0.2) (layer "F.Cu") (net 3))
 (segment (start 124.46 69.215) (end 128.27 73.025) (width 0.2) (layer "F.Cu") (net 3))
 (segment (start 95.434 70.301) (end 90.17 75.565) (width 0.2) (layer "F.Cu") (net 3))
 (segment (start 113.03 64.135) (end 109.22 64.135) (width 0.2) (layer "F.Cu") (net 4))
 (segment (start 109.22 64.135) (end 107.95 65.405) (width 0.2) (layer "F.Cu") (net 4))
 (segment (start 132.08 64.135) (end 129.54 64.135) (width 0.2) (layer "B.Cu") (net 6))
 (segment (start 129.54 64.135) (end 128.27 65.405) (width 0.2) (layer "B.Cu") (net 6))
 (segment (start 93.98 83.185) (end 90.17 83.185) (width 0.2) (layer "B.Cu") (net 20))
 (segment (start 113.03 83.185) (end 109.22 83.185) (width 0.2) (layer "B.Cu") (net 12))
 (segment (start 132.08 83.185) (end 128.27 83.185) (width 0.2) (layer "B.Cu") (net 19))
 (segment (start 130.139854 72.354854) (end 130.139854 84.062436) (width 0.2) (layer "F.Cu") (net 1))
 (segment (start 106.68 116.205) (end 109.22 113.665) (width 0.2) (layer "F.Cu") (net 1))
 (segment (start 128.49507 85.70722) (end 128.49507 94.38993) (width 0.2) (layer "F.Cu") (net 1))
 (segment (start 118.11 53.975) (end 118.11 56.515) (width 0.2) (layer "F.Cu") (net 1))
 (segment (start 109.22 125.095) (end 106.68 122.555) (width 0.2) (layer "F.Cu") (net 1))
 (segment (start 125.73 64.135) (end 125.73 67.945) (width 0.2) (layer "F.Cu") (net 1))
 (segment (start 128.49507 94.38993) (end 109.22 113.665) (width 0.2) (layer "F.Cu") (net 1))
 (segment (start 106.68 122.555) (end 106.68 116.205) (width 0.2) (layer "F.Cu") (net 1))
 (segment (start 125.73 67.945) (end 130.139854 72.354854) (width 0.2) (layer "F.Cu") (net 1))
 (segment (start 109.22 132.715) (end 109.22 125.095) (width 0.2) (layer "F.Cu") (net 1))
 (segment (start 118.11 56.515) (end 125.73 64.135) (width 0.2) (layer "F.Cu") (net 1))
 (segment (start 130.139854 84.062436) (end 128.49507 85.70722) (width 0.2) (layer "F.Cu") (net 1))
 (segment (start 132.908335 87.506886) (end 132.908335 84.948279) (width 0.2) (layer "F.Cu") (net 7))
 (segment (start 126.723382 66.398382) (end 126.723382 60.048382) (width 0.2) (layer "F.Cu") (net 7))
 (segment (start 124.968 132.08) (end 124.968 125.476) (width 0.2) (layer "F.Cu") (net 7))
 (segment (start 124.968 125.476) (end 128.27 122.174) (width 0.2) (layer "F.Cu") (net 7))
 (segment (start 133.913502 83.943112) (end 133.913502 82.034311) (width 0.2) (layer "F.Cu") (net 7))
 (segment (start 126.723382 60.048382) (end 120.65 53.975) (width 0.2) (layer "F.Cu") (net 7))
 (segment (start 128.27 96.391821) (end 129.54 95.121821) (width 0.2) (layer "F.Cu") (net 7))
 (segment (start 132.938795 81.059604) (end 132.938795 72.613795) (width 0.2) (layer "F.Cu") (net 7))
 (segment (start 132.938795 72.613795) (end 126.723382 66.398382) (width 0.2) (layer "F.Cu") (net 7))
 (segment (start 133.913502 82.034311) (end 132.938795 81.059604) (width 0.2) (layer "F.Cu") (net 7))
 (segment (start 132.908335 84.948279) (end 133.913502 83.943112) (width 0.2) (layer "F.Cu") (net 7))
 (segment (start 129.54 90.875221) (end 132.908335 87.506886) (width 0.2) (layer "F.Cu") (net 7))
 (segment (start 128.27 122.174) (end 128.27 96.391821) (width 0.2) (layer "F.Cu") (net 7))
 (segment (start 129.54 95.121821) (end 129.54 90.875221) (width 0.2) (layer "F.Cu") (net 7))
 (segment (start 123.698 133.985) (end 91.44 133.985) (width 0.2) (layer "B.Cu") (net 7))
 (segment (start 91.44 133.985) (end 90.17 132.715) (width 0.2) (layer "B.Cu") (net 7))
 (segment (start 124.968 132.715) (end 123.698 133.985) (width 0.2) (layer "B.Cu") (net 7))
 (segment (start 93.98 140.335) (end 90.17 140.335) (width 0.2) (layer "B.Cu") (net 13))
 (segment (start 113.03 140.335) (end 109.22 140.335) (width 0.2) (layer "B.Cu") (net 22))
 (segment (start 132.08 140.335) (end 125.603 140.335) (width 0.2) (layer "B.Cu") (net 23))
 (segment (start 104.1046 106.553) (end 98.517 106.553) (width 0.2) (layer "F.Cu") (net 16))
 (segment (start 98.4705 115.375) (end 100.1125 115.375) (width 0.2) (layer "F.Cu") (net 16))
 (segment (start 133.35 41.275) (end 131.580464 39.505464) (width 0.2) (layer "F.Cu") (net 16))
 (segment (start 88.414935 105.319435) (end 94.10025 111.00475) (width 0.2) (layer "F.Cu") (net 16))
 (segment (start 102.099536 39.505464) (end 88.414935 53.190065) (width 0.2) (layer "F.Cu") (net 16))
 (segment (start 94.10025 111.00475) (end 98.4705 115.375) (width 0.2) (layer "F.Cu") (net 16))
 (segment (start 104.1146 106.543) (end 104.1046 106.553) (width 0.2) (layer "F.Cu") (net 16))
 (segment (start 94.10025 110.96975) (end 94.10025 111.00475) (width 0.2) (layer "F.Cu") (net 16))
 (segment (start 88.414935 53.190065) (end 88.414935 105.319435) (width 0.2) (layer "F.Cu") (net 16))
 (segment (start 131.580464 39.505464) (end 102.099536 39.505464) (width 0.2) (layer "F.Cu") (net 16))
 (segment (start 98.517 106.553) (end 94.10025 110.96975) (width 0.2) (layer "F.Cu") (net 16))
 (segment (start 107.055559 127.376059) (end 125.766441 127.376059) (width 0.2) (layer "B.Cu") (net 16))
 (segment (start 100.1125 120.433) (end 107.055559 127.376059) (width 0.2) (layer "B.Cu") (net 16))
 (segment (start 100.1125 115.375) (end 100.1125 120.433) (width 0.2) (layer "B.Cu") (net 16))
 (segment (start 125.766441 127.376059) (end 133.5675 119.575) (width 0.2) (layer "B.Cu") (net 16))
 (segment (start 143.305741 53.770741) (end 143.305741 113.836759) (width 0.2) (layer "F.Cu") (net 15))
 (segment (start 143.305741 113.836759) (end 137.5675 119.575) (width 0.2) (layer "F.Cu") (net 15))
 (segment (start 130.81 41.275) (end 143.305741 53.770741) (width 0.2) (layer "F.Cu") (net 15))
 (segment (start 128.989721 128.152779) (end 106.202018 128.152779) (width 0.2) (layer "B.Cu") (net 15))
 (segment (start 104.1146 109.083) (end 102.4045 109.083) (width 0.2) (layer "B.Cu") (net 15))
 (segment (start 102.4045 109.083) (end 96.1125 115.375) (width 0.2) (layer "B.Cu") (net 15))
 (segment (start 106.202018 128.152779) (end 96.1125 118.063261) (width 0.2) (layer "B.Cu") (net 15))
 (segment (start 96.1125 118.063261) (end 96.1125 115.375) (width 0.2) (layer "B.Cu") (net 15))
 (segment (start 137.5675 119.575) (end 128.989721 128.152779) (width 0.2) (layer "B.Cu") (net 15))
 (segment (start 142.651714 104.790786) (end 132.0675 115.375) (width 0.2) (layer "F.Cu") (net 17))
 (segment (start 128.27 41.275) (end 142.651714 55.656714) (width 0.2) (layer "F.Cu") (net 17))
 (segment (start 142.651714 55.656714) (end 142.651714 104.790786) (width 0.2) (layer "F.Cu") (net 17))
 (segment (start 108.613994 126.576494) (end 121.599347 126.576494) (width 0.2) (layer "B.Cu") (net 17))
 (segment (start 107.0102 114.1773) (end 101.6125 119.575) (width 0.2) (layer "B.Cu") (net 17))
 (segment (start 132.0675 116.108341) (end 132.0675 115.375) (width 0.2) (layer "B.Cu") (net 17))
 (segment (start 101.6125 119.575) (end 108.613994 126.576494) (width 0.2) (layer "B.Cu") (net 17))
 (segment (start 104.1146 104.003) (end 107.0102 106.8986) (width 0.2) (layer "B.Cu") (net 17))
 (segment (start 121.599347 126.576494) (end 132.0675 116.108341) (width 0.2) (layer "B.Cu") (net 17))
 (segment (start 107.0102 106.8986) (end 107.0102 114.1773) (width 0.2) (layer "B.Cu") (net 17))
 (segment (start 93.1125 115.375) (end 93.1125 106.8775) (width 0.2) (layer "B.Cu") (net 18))
 (segment (start 93.1125 116.6075) (end 105.41 128.905) (width 0.2) (layer "B.Cu") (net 18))
 (segment (start 125.73 41.275) (end 142.349158 57.894158) (width 0.2) (layer "B.Cu") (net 18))
 (segment (start 142.349158 57.894158) (end 142.349158 114.701842) (width 0.2) (layer "B.Cu") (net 18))
 (segment (start 105.41 128.905) (end 131.2375 128.905) (width 0.2) (layer "B.Cu") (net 18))
 (segment (start 104.0992 101.4476) (end 104.1146 101.463) (width 0.2) (layer "B.Cu") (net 18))
 (segment (start 98.5424 101.4476) (end 104.0992 101.4476) (width 0.2) (layer "B.Cu") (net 18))
 (segment (start 140.5675 116.4835) (end 140.5675 119.575) (width 0.2) (layer "B.Cu") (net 18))
 (segment (start 131.2375 128.905) (end 140.5675 119.575) (width 0.2) (layer "B.Cu") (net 18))
 (segment (start 93.1125 115.375) (end 93.1125 116.6075) (width 0.2) (layer "B.Cu") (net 18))
 (segment (start 93.1125 106.8775) (end 98.5424 101.4476) (width 0.2) (layer "B.Cu") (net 18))
 (segment (start 142.349158 114.701842) (end 140.5675 116.4835) (width 0.2) (layer "B.Cu") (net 18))
 (segment (start 119.38 61.595) (end 100.33 61.595) (width 0.2) (layer "F.Cu") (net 9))
 (segment (start 105.41 53.975) (end 105.41 56.515) (width 0.2) (layer "B.Cu") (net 9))
 (segment (start 105.41 56.515) (end 100.33 61.595) (width 0.2) (layer "B.Cu") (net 9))
 (segment (start 107.709529 137.795) (end 100.33 137.795) (width 0.2) (layer "F.Cu") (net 5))
 (segment (start 119.38 118.745) (end 119.77177 119.13677) (width 0.2) (layer "F.Cu") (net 5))
 (segment (start 119.77177 125.732759) (end 107.709529 137.795) (width 0.2) (layer "F.Cu") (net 5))
 (segment (start 119.77177 119.13677) (end 119.77177 125.732759) (width 0.2) (layer "F.Cu") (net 5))
 (segment (start 140.490261 78.895261) (end 140.490261 82.394739) (width 0.2) (layer "B.Cu") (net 5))
 (segment (start 107.95 53.975) (end 107.95 55.245) (width 0.2) (layer "B.Cu") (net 5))
 (segment (start 139.096734 91.408266) (end 124.46 106.045) (width 0.2) (layer "B.Cu") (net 5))
 (segment (start 104.074 76.901) (end 100.33 80.645) (width 0.2) (layer "B.Cu") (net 5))
 (segment (start 104.074 59.121) (end 104.074 76.901) (width 0.2) (layer "B.Cu") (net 5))
 (segment (start 124.46 106.045) (end 119.38 106.045) (width 0.2) (layer "B.Cu") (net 5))
 (segment (start 140.490261 82.394739) (end 139.096734 83.788266) (width 0.2) (layer "B.Cu") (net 5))
 (segment (start 139.005355 77.410355) (end 140.490261 78.895261) (width 0.2) (layer "B.Cu") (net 5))
 (segment (start 100.33 86.995) (end 119.38 106.045) (width 0.2) (layer "B.Cu") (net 5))
 (segment (start 100.33 80.645) (end 100.33 86.995) (width 0.2) (layer "B.Cu") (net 5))
 (segment (start 139.005355 62.170355) (end 139.005355 77.410355) (width 0.2) (layer "B.Cu") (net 5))
 (segment (start 107.95 55.245) (end 104.074 59.121) (width 0.2) (layer "B.Cu") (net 5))
 (segment (start 119.38 106.045) (end 119.38 118.745) (width 0.2) (layer "B.Cu") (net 5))
 (segment (start 139.096734 83.788266) (end 139.096734 91.408266) (width 0.2) (layer "B.Cu") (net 5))
 (segment (start 138.43 61.595) (end 139.005355 62.170355) (width 0.2) (layer "B.Cu") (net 5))
 (segment (start 138.43 86.514059) (end 138.43 80.645) (width 0.2) (layer "F.Cu") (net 14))
 (segment (start 130.81 94.134059) (end 138.43 86.514059) (width 0.2) (layer "F.Cu") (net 14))
 (segment (start 129.54 97.155) (end 130.81 95.885) (width 0.2) (layer "F.Cu") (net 14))
 (segment (start 129.54 128.905) (end 129.54 97.155) (width 0.2) (layer "F.Cu") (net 14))
 (segment (start 138.43 137.795) (end 129.54 128.905) (width 0.2) (layer "F.Cu") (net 14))
 (segment (start 130.81 95.885) (end 130.81 94.134059) (width 0.2) (layer "F.Cu") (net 14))
 (segment (start 110.091935 53.975) (end 110.49 53.975) (width 0.2) (layer "B.Cu") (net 14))
 (segment (start 119.38 137.795) (end 138.43 137.795) (width 0.2) (layer "B.Cu") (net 14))
 (segment (start 110.49 53.975) (end 109.960435 54.504565) (width 0.2) (layer "B.Cu") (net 14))
 (segment (start 106.68 57.386935) (end 110.091935 53.975) (width 0.2) (layer "B.Cu") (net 14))
 (segment (start 119.38 80.645) (end 111.76 80.645) (width 0.2) (layer "B.Cu") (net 14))
 (segment (start 106.68 75.565) (end 106.68 57.386935) (width 0.2) (layer "B.Cu") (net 14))
 (segment (start 138.43 80.645) (end 119.38 80.645) (width 0.2) (layer "B.Cu") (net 14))
 (segment (start 111.76 80.645) (end 106.68 75.565) (width 0.2) (layer "B.Cu") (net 14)))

